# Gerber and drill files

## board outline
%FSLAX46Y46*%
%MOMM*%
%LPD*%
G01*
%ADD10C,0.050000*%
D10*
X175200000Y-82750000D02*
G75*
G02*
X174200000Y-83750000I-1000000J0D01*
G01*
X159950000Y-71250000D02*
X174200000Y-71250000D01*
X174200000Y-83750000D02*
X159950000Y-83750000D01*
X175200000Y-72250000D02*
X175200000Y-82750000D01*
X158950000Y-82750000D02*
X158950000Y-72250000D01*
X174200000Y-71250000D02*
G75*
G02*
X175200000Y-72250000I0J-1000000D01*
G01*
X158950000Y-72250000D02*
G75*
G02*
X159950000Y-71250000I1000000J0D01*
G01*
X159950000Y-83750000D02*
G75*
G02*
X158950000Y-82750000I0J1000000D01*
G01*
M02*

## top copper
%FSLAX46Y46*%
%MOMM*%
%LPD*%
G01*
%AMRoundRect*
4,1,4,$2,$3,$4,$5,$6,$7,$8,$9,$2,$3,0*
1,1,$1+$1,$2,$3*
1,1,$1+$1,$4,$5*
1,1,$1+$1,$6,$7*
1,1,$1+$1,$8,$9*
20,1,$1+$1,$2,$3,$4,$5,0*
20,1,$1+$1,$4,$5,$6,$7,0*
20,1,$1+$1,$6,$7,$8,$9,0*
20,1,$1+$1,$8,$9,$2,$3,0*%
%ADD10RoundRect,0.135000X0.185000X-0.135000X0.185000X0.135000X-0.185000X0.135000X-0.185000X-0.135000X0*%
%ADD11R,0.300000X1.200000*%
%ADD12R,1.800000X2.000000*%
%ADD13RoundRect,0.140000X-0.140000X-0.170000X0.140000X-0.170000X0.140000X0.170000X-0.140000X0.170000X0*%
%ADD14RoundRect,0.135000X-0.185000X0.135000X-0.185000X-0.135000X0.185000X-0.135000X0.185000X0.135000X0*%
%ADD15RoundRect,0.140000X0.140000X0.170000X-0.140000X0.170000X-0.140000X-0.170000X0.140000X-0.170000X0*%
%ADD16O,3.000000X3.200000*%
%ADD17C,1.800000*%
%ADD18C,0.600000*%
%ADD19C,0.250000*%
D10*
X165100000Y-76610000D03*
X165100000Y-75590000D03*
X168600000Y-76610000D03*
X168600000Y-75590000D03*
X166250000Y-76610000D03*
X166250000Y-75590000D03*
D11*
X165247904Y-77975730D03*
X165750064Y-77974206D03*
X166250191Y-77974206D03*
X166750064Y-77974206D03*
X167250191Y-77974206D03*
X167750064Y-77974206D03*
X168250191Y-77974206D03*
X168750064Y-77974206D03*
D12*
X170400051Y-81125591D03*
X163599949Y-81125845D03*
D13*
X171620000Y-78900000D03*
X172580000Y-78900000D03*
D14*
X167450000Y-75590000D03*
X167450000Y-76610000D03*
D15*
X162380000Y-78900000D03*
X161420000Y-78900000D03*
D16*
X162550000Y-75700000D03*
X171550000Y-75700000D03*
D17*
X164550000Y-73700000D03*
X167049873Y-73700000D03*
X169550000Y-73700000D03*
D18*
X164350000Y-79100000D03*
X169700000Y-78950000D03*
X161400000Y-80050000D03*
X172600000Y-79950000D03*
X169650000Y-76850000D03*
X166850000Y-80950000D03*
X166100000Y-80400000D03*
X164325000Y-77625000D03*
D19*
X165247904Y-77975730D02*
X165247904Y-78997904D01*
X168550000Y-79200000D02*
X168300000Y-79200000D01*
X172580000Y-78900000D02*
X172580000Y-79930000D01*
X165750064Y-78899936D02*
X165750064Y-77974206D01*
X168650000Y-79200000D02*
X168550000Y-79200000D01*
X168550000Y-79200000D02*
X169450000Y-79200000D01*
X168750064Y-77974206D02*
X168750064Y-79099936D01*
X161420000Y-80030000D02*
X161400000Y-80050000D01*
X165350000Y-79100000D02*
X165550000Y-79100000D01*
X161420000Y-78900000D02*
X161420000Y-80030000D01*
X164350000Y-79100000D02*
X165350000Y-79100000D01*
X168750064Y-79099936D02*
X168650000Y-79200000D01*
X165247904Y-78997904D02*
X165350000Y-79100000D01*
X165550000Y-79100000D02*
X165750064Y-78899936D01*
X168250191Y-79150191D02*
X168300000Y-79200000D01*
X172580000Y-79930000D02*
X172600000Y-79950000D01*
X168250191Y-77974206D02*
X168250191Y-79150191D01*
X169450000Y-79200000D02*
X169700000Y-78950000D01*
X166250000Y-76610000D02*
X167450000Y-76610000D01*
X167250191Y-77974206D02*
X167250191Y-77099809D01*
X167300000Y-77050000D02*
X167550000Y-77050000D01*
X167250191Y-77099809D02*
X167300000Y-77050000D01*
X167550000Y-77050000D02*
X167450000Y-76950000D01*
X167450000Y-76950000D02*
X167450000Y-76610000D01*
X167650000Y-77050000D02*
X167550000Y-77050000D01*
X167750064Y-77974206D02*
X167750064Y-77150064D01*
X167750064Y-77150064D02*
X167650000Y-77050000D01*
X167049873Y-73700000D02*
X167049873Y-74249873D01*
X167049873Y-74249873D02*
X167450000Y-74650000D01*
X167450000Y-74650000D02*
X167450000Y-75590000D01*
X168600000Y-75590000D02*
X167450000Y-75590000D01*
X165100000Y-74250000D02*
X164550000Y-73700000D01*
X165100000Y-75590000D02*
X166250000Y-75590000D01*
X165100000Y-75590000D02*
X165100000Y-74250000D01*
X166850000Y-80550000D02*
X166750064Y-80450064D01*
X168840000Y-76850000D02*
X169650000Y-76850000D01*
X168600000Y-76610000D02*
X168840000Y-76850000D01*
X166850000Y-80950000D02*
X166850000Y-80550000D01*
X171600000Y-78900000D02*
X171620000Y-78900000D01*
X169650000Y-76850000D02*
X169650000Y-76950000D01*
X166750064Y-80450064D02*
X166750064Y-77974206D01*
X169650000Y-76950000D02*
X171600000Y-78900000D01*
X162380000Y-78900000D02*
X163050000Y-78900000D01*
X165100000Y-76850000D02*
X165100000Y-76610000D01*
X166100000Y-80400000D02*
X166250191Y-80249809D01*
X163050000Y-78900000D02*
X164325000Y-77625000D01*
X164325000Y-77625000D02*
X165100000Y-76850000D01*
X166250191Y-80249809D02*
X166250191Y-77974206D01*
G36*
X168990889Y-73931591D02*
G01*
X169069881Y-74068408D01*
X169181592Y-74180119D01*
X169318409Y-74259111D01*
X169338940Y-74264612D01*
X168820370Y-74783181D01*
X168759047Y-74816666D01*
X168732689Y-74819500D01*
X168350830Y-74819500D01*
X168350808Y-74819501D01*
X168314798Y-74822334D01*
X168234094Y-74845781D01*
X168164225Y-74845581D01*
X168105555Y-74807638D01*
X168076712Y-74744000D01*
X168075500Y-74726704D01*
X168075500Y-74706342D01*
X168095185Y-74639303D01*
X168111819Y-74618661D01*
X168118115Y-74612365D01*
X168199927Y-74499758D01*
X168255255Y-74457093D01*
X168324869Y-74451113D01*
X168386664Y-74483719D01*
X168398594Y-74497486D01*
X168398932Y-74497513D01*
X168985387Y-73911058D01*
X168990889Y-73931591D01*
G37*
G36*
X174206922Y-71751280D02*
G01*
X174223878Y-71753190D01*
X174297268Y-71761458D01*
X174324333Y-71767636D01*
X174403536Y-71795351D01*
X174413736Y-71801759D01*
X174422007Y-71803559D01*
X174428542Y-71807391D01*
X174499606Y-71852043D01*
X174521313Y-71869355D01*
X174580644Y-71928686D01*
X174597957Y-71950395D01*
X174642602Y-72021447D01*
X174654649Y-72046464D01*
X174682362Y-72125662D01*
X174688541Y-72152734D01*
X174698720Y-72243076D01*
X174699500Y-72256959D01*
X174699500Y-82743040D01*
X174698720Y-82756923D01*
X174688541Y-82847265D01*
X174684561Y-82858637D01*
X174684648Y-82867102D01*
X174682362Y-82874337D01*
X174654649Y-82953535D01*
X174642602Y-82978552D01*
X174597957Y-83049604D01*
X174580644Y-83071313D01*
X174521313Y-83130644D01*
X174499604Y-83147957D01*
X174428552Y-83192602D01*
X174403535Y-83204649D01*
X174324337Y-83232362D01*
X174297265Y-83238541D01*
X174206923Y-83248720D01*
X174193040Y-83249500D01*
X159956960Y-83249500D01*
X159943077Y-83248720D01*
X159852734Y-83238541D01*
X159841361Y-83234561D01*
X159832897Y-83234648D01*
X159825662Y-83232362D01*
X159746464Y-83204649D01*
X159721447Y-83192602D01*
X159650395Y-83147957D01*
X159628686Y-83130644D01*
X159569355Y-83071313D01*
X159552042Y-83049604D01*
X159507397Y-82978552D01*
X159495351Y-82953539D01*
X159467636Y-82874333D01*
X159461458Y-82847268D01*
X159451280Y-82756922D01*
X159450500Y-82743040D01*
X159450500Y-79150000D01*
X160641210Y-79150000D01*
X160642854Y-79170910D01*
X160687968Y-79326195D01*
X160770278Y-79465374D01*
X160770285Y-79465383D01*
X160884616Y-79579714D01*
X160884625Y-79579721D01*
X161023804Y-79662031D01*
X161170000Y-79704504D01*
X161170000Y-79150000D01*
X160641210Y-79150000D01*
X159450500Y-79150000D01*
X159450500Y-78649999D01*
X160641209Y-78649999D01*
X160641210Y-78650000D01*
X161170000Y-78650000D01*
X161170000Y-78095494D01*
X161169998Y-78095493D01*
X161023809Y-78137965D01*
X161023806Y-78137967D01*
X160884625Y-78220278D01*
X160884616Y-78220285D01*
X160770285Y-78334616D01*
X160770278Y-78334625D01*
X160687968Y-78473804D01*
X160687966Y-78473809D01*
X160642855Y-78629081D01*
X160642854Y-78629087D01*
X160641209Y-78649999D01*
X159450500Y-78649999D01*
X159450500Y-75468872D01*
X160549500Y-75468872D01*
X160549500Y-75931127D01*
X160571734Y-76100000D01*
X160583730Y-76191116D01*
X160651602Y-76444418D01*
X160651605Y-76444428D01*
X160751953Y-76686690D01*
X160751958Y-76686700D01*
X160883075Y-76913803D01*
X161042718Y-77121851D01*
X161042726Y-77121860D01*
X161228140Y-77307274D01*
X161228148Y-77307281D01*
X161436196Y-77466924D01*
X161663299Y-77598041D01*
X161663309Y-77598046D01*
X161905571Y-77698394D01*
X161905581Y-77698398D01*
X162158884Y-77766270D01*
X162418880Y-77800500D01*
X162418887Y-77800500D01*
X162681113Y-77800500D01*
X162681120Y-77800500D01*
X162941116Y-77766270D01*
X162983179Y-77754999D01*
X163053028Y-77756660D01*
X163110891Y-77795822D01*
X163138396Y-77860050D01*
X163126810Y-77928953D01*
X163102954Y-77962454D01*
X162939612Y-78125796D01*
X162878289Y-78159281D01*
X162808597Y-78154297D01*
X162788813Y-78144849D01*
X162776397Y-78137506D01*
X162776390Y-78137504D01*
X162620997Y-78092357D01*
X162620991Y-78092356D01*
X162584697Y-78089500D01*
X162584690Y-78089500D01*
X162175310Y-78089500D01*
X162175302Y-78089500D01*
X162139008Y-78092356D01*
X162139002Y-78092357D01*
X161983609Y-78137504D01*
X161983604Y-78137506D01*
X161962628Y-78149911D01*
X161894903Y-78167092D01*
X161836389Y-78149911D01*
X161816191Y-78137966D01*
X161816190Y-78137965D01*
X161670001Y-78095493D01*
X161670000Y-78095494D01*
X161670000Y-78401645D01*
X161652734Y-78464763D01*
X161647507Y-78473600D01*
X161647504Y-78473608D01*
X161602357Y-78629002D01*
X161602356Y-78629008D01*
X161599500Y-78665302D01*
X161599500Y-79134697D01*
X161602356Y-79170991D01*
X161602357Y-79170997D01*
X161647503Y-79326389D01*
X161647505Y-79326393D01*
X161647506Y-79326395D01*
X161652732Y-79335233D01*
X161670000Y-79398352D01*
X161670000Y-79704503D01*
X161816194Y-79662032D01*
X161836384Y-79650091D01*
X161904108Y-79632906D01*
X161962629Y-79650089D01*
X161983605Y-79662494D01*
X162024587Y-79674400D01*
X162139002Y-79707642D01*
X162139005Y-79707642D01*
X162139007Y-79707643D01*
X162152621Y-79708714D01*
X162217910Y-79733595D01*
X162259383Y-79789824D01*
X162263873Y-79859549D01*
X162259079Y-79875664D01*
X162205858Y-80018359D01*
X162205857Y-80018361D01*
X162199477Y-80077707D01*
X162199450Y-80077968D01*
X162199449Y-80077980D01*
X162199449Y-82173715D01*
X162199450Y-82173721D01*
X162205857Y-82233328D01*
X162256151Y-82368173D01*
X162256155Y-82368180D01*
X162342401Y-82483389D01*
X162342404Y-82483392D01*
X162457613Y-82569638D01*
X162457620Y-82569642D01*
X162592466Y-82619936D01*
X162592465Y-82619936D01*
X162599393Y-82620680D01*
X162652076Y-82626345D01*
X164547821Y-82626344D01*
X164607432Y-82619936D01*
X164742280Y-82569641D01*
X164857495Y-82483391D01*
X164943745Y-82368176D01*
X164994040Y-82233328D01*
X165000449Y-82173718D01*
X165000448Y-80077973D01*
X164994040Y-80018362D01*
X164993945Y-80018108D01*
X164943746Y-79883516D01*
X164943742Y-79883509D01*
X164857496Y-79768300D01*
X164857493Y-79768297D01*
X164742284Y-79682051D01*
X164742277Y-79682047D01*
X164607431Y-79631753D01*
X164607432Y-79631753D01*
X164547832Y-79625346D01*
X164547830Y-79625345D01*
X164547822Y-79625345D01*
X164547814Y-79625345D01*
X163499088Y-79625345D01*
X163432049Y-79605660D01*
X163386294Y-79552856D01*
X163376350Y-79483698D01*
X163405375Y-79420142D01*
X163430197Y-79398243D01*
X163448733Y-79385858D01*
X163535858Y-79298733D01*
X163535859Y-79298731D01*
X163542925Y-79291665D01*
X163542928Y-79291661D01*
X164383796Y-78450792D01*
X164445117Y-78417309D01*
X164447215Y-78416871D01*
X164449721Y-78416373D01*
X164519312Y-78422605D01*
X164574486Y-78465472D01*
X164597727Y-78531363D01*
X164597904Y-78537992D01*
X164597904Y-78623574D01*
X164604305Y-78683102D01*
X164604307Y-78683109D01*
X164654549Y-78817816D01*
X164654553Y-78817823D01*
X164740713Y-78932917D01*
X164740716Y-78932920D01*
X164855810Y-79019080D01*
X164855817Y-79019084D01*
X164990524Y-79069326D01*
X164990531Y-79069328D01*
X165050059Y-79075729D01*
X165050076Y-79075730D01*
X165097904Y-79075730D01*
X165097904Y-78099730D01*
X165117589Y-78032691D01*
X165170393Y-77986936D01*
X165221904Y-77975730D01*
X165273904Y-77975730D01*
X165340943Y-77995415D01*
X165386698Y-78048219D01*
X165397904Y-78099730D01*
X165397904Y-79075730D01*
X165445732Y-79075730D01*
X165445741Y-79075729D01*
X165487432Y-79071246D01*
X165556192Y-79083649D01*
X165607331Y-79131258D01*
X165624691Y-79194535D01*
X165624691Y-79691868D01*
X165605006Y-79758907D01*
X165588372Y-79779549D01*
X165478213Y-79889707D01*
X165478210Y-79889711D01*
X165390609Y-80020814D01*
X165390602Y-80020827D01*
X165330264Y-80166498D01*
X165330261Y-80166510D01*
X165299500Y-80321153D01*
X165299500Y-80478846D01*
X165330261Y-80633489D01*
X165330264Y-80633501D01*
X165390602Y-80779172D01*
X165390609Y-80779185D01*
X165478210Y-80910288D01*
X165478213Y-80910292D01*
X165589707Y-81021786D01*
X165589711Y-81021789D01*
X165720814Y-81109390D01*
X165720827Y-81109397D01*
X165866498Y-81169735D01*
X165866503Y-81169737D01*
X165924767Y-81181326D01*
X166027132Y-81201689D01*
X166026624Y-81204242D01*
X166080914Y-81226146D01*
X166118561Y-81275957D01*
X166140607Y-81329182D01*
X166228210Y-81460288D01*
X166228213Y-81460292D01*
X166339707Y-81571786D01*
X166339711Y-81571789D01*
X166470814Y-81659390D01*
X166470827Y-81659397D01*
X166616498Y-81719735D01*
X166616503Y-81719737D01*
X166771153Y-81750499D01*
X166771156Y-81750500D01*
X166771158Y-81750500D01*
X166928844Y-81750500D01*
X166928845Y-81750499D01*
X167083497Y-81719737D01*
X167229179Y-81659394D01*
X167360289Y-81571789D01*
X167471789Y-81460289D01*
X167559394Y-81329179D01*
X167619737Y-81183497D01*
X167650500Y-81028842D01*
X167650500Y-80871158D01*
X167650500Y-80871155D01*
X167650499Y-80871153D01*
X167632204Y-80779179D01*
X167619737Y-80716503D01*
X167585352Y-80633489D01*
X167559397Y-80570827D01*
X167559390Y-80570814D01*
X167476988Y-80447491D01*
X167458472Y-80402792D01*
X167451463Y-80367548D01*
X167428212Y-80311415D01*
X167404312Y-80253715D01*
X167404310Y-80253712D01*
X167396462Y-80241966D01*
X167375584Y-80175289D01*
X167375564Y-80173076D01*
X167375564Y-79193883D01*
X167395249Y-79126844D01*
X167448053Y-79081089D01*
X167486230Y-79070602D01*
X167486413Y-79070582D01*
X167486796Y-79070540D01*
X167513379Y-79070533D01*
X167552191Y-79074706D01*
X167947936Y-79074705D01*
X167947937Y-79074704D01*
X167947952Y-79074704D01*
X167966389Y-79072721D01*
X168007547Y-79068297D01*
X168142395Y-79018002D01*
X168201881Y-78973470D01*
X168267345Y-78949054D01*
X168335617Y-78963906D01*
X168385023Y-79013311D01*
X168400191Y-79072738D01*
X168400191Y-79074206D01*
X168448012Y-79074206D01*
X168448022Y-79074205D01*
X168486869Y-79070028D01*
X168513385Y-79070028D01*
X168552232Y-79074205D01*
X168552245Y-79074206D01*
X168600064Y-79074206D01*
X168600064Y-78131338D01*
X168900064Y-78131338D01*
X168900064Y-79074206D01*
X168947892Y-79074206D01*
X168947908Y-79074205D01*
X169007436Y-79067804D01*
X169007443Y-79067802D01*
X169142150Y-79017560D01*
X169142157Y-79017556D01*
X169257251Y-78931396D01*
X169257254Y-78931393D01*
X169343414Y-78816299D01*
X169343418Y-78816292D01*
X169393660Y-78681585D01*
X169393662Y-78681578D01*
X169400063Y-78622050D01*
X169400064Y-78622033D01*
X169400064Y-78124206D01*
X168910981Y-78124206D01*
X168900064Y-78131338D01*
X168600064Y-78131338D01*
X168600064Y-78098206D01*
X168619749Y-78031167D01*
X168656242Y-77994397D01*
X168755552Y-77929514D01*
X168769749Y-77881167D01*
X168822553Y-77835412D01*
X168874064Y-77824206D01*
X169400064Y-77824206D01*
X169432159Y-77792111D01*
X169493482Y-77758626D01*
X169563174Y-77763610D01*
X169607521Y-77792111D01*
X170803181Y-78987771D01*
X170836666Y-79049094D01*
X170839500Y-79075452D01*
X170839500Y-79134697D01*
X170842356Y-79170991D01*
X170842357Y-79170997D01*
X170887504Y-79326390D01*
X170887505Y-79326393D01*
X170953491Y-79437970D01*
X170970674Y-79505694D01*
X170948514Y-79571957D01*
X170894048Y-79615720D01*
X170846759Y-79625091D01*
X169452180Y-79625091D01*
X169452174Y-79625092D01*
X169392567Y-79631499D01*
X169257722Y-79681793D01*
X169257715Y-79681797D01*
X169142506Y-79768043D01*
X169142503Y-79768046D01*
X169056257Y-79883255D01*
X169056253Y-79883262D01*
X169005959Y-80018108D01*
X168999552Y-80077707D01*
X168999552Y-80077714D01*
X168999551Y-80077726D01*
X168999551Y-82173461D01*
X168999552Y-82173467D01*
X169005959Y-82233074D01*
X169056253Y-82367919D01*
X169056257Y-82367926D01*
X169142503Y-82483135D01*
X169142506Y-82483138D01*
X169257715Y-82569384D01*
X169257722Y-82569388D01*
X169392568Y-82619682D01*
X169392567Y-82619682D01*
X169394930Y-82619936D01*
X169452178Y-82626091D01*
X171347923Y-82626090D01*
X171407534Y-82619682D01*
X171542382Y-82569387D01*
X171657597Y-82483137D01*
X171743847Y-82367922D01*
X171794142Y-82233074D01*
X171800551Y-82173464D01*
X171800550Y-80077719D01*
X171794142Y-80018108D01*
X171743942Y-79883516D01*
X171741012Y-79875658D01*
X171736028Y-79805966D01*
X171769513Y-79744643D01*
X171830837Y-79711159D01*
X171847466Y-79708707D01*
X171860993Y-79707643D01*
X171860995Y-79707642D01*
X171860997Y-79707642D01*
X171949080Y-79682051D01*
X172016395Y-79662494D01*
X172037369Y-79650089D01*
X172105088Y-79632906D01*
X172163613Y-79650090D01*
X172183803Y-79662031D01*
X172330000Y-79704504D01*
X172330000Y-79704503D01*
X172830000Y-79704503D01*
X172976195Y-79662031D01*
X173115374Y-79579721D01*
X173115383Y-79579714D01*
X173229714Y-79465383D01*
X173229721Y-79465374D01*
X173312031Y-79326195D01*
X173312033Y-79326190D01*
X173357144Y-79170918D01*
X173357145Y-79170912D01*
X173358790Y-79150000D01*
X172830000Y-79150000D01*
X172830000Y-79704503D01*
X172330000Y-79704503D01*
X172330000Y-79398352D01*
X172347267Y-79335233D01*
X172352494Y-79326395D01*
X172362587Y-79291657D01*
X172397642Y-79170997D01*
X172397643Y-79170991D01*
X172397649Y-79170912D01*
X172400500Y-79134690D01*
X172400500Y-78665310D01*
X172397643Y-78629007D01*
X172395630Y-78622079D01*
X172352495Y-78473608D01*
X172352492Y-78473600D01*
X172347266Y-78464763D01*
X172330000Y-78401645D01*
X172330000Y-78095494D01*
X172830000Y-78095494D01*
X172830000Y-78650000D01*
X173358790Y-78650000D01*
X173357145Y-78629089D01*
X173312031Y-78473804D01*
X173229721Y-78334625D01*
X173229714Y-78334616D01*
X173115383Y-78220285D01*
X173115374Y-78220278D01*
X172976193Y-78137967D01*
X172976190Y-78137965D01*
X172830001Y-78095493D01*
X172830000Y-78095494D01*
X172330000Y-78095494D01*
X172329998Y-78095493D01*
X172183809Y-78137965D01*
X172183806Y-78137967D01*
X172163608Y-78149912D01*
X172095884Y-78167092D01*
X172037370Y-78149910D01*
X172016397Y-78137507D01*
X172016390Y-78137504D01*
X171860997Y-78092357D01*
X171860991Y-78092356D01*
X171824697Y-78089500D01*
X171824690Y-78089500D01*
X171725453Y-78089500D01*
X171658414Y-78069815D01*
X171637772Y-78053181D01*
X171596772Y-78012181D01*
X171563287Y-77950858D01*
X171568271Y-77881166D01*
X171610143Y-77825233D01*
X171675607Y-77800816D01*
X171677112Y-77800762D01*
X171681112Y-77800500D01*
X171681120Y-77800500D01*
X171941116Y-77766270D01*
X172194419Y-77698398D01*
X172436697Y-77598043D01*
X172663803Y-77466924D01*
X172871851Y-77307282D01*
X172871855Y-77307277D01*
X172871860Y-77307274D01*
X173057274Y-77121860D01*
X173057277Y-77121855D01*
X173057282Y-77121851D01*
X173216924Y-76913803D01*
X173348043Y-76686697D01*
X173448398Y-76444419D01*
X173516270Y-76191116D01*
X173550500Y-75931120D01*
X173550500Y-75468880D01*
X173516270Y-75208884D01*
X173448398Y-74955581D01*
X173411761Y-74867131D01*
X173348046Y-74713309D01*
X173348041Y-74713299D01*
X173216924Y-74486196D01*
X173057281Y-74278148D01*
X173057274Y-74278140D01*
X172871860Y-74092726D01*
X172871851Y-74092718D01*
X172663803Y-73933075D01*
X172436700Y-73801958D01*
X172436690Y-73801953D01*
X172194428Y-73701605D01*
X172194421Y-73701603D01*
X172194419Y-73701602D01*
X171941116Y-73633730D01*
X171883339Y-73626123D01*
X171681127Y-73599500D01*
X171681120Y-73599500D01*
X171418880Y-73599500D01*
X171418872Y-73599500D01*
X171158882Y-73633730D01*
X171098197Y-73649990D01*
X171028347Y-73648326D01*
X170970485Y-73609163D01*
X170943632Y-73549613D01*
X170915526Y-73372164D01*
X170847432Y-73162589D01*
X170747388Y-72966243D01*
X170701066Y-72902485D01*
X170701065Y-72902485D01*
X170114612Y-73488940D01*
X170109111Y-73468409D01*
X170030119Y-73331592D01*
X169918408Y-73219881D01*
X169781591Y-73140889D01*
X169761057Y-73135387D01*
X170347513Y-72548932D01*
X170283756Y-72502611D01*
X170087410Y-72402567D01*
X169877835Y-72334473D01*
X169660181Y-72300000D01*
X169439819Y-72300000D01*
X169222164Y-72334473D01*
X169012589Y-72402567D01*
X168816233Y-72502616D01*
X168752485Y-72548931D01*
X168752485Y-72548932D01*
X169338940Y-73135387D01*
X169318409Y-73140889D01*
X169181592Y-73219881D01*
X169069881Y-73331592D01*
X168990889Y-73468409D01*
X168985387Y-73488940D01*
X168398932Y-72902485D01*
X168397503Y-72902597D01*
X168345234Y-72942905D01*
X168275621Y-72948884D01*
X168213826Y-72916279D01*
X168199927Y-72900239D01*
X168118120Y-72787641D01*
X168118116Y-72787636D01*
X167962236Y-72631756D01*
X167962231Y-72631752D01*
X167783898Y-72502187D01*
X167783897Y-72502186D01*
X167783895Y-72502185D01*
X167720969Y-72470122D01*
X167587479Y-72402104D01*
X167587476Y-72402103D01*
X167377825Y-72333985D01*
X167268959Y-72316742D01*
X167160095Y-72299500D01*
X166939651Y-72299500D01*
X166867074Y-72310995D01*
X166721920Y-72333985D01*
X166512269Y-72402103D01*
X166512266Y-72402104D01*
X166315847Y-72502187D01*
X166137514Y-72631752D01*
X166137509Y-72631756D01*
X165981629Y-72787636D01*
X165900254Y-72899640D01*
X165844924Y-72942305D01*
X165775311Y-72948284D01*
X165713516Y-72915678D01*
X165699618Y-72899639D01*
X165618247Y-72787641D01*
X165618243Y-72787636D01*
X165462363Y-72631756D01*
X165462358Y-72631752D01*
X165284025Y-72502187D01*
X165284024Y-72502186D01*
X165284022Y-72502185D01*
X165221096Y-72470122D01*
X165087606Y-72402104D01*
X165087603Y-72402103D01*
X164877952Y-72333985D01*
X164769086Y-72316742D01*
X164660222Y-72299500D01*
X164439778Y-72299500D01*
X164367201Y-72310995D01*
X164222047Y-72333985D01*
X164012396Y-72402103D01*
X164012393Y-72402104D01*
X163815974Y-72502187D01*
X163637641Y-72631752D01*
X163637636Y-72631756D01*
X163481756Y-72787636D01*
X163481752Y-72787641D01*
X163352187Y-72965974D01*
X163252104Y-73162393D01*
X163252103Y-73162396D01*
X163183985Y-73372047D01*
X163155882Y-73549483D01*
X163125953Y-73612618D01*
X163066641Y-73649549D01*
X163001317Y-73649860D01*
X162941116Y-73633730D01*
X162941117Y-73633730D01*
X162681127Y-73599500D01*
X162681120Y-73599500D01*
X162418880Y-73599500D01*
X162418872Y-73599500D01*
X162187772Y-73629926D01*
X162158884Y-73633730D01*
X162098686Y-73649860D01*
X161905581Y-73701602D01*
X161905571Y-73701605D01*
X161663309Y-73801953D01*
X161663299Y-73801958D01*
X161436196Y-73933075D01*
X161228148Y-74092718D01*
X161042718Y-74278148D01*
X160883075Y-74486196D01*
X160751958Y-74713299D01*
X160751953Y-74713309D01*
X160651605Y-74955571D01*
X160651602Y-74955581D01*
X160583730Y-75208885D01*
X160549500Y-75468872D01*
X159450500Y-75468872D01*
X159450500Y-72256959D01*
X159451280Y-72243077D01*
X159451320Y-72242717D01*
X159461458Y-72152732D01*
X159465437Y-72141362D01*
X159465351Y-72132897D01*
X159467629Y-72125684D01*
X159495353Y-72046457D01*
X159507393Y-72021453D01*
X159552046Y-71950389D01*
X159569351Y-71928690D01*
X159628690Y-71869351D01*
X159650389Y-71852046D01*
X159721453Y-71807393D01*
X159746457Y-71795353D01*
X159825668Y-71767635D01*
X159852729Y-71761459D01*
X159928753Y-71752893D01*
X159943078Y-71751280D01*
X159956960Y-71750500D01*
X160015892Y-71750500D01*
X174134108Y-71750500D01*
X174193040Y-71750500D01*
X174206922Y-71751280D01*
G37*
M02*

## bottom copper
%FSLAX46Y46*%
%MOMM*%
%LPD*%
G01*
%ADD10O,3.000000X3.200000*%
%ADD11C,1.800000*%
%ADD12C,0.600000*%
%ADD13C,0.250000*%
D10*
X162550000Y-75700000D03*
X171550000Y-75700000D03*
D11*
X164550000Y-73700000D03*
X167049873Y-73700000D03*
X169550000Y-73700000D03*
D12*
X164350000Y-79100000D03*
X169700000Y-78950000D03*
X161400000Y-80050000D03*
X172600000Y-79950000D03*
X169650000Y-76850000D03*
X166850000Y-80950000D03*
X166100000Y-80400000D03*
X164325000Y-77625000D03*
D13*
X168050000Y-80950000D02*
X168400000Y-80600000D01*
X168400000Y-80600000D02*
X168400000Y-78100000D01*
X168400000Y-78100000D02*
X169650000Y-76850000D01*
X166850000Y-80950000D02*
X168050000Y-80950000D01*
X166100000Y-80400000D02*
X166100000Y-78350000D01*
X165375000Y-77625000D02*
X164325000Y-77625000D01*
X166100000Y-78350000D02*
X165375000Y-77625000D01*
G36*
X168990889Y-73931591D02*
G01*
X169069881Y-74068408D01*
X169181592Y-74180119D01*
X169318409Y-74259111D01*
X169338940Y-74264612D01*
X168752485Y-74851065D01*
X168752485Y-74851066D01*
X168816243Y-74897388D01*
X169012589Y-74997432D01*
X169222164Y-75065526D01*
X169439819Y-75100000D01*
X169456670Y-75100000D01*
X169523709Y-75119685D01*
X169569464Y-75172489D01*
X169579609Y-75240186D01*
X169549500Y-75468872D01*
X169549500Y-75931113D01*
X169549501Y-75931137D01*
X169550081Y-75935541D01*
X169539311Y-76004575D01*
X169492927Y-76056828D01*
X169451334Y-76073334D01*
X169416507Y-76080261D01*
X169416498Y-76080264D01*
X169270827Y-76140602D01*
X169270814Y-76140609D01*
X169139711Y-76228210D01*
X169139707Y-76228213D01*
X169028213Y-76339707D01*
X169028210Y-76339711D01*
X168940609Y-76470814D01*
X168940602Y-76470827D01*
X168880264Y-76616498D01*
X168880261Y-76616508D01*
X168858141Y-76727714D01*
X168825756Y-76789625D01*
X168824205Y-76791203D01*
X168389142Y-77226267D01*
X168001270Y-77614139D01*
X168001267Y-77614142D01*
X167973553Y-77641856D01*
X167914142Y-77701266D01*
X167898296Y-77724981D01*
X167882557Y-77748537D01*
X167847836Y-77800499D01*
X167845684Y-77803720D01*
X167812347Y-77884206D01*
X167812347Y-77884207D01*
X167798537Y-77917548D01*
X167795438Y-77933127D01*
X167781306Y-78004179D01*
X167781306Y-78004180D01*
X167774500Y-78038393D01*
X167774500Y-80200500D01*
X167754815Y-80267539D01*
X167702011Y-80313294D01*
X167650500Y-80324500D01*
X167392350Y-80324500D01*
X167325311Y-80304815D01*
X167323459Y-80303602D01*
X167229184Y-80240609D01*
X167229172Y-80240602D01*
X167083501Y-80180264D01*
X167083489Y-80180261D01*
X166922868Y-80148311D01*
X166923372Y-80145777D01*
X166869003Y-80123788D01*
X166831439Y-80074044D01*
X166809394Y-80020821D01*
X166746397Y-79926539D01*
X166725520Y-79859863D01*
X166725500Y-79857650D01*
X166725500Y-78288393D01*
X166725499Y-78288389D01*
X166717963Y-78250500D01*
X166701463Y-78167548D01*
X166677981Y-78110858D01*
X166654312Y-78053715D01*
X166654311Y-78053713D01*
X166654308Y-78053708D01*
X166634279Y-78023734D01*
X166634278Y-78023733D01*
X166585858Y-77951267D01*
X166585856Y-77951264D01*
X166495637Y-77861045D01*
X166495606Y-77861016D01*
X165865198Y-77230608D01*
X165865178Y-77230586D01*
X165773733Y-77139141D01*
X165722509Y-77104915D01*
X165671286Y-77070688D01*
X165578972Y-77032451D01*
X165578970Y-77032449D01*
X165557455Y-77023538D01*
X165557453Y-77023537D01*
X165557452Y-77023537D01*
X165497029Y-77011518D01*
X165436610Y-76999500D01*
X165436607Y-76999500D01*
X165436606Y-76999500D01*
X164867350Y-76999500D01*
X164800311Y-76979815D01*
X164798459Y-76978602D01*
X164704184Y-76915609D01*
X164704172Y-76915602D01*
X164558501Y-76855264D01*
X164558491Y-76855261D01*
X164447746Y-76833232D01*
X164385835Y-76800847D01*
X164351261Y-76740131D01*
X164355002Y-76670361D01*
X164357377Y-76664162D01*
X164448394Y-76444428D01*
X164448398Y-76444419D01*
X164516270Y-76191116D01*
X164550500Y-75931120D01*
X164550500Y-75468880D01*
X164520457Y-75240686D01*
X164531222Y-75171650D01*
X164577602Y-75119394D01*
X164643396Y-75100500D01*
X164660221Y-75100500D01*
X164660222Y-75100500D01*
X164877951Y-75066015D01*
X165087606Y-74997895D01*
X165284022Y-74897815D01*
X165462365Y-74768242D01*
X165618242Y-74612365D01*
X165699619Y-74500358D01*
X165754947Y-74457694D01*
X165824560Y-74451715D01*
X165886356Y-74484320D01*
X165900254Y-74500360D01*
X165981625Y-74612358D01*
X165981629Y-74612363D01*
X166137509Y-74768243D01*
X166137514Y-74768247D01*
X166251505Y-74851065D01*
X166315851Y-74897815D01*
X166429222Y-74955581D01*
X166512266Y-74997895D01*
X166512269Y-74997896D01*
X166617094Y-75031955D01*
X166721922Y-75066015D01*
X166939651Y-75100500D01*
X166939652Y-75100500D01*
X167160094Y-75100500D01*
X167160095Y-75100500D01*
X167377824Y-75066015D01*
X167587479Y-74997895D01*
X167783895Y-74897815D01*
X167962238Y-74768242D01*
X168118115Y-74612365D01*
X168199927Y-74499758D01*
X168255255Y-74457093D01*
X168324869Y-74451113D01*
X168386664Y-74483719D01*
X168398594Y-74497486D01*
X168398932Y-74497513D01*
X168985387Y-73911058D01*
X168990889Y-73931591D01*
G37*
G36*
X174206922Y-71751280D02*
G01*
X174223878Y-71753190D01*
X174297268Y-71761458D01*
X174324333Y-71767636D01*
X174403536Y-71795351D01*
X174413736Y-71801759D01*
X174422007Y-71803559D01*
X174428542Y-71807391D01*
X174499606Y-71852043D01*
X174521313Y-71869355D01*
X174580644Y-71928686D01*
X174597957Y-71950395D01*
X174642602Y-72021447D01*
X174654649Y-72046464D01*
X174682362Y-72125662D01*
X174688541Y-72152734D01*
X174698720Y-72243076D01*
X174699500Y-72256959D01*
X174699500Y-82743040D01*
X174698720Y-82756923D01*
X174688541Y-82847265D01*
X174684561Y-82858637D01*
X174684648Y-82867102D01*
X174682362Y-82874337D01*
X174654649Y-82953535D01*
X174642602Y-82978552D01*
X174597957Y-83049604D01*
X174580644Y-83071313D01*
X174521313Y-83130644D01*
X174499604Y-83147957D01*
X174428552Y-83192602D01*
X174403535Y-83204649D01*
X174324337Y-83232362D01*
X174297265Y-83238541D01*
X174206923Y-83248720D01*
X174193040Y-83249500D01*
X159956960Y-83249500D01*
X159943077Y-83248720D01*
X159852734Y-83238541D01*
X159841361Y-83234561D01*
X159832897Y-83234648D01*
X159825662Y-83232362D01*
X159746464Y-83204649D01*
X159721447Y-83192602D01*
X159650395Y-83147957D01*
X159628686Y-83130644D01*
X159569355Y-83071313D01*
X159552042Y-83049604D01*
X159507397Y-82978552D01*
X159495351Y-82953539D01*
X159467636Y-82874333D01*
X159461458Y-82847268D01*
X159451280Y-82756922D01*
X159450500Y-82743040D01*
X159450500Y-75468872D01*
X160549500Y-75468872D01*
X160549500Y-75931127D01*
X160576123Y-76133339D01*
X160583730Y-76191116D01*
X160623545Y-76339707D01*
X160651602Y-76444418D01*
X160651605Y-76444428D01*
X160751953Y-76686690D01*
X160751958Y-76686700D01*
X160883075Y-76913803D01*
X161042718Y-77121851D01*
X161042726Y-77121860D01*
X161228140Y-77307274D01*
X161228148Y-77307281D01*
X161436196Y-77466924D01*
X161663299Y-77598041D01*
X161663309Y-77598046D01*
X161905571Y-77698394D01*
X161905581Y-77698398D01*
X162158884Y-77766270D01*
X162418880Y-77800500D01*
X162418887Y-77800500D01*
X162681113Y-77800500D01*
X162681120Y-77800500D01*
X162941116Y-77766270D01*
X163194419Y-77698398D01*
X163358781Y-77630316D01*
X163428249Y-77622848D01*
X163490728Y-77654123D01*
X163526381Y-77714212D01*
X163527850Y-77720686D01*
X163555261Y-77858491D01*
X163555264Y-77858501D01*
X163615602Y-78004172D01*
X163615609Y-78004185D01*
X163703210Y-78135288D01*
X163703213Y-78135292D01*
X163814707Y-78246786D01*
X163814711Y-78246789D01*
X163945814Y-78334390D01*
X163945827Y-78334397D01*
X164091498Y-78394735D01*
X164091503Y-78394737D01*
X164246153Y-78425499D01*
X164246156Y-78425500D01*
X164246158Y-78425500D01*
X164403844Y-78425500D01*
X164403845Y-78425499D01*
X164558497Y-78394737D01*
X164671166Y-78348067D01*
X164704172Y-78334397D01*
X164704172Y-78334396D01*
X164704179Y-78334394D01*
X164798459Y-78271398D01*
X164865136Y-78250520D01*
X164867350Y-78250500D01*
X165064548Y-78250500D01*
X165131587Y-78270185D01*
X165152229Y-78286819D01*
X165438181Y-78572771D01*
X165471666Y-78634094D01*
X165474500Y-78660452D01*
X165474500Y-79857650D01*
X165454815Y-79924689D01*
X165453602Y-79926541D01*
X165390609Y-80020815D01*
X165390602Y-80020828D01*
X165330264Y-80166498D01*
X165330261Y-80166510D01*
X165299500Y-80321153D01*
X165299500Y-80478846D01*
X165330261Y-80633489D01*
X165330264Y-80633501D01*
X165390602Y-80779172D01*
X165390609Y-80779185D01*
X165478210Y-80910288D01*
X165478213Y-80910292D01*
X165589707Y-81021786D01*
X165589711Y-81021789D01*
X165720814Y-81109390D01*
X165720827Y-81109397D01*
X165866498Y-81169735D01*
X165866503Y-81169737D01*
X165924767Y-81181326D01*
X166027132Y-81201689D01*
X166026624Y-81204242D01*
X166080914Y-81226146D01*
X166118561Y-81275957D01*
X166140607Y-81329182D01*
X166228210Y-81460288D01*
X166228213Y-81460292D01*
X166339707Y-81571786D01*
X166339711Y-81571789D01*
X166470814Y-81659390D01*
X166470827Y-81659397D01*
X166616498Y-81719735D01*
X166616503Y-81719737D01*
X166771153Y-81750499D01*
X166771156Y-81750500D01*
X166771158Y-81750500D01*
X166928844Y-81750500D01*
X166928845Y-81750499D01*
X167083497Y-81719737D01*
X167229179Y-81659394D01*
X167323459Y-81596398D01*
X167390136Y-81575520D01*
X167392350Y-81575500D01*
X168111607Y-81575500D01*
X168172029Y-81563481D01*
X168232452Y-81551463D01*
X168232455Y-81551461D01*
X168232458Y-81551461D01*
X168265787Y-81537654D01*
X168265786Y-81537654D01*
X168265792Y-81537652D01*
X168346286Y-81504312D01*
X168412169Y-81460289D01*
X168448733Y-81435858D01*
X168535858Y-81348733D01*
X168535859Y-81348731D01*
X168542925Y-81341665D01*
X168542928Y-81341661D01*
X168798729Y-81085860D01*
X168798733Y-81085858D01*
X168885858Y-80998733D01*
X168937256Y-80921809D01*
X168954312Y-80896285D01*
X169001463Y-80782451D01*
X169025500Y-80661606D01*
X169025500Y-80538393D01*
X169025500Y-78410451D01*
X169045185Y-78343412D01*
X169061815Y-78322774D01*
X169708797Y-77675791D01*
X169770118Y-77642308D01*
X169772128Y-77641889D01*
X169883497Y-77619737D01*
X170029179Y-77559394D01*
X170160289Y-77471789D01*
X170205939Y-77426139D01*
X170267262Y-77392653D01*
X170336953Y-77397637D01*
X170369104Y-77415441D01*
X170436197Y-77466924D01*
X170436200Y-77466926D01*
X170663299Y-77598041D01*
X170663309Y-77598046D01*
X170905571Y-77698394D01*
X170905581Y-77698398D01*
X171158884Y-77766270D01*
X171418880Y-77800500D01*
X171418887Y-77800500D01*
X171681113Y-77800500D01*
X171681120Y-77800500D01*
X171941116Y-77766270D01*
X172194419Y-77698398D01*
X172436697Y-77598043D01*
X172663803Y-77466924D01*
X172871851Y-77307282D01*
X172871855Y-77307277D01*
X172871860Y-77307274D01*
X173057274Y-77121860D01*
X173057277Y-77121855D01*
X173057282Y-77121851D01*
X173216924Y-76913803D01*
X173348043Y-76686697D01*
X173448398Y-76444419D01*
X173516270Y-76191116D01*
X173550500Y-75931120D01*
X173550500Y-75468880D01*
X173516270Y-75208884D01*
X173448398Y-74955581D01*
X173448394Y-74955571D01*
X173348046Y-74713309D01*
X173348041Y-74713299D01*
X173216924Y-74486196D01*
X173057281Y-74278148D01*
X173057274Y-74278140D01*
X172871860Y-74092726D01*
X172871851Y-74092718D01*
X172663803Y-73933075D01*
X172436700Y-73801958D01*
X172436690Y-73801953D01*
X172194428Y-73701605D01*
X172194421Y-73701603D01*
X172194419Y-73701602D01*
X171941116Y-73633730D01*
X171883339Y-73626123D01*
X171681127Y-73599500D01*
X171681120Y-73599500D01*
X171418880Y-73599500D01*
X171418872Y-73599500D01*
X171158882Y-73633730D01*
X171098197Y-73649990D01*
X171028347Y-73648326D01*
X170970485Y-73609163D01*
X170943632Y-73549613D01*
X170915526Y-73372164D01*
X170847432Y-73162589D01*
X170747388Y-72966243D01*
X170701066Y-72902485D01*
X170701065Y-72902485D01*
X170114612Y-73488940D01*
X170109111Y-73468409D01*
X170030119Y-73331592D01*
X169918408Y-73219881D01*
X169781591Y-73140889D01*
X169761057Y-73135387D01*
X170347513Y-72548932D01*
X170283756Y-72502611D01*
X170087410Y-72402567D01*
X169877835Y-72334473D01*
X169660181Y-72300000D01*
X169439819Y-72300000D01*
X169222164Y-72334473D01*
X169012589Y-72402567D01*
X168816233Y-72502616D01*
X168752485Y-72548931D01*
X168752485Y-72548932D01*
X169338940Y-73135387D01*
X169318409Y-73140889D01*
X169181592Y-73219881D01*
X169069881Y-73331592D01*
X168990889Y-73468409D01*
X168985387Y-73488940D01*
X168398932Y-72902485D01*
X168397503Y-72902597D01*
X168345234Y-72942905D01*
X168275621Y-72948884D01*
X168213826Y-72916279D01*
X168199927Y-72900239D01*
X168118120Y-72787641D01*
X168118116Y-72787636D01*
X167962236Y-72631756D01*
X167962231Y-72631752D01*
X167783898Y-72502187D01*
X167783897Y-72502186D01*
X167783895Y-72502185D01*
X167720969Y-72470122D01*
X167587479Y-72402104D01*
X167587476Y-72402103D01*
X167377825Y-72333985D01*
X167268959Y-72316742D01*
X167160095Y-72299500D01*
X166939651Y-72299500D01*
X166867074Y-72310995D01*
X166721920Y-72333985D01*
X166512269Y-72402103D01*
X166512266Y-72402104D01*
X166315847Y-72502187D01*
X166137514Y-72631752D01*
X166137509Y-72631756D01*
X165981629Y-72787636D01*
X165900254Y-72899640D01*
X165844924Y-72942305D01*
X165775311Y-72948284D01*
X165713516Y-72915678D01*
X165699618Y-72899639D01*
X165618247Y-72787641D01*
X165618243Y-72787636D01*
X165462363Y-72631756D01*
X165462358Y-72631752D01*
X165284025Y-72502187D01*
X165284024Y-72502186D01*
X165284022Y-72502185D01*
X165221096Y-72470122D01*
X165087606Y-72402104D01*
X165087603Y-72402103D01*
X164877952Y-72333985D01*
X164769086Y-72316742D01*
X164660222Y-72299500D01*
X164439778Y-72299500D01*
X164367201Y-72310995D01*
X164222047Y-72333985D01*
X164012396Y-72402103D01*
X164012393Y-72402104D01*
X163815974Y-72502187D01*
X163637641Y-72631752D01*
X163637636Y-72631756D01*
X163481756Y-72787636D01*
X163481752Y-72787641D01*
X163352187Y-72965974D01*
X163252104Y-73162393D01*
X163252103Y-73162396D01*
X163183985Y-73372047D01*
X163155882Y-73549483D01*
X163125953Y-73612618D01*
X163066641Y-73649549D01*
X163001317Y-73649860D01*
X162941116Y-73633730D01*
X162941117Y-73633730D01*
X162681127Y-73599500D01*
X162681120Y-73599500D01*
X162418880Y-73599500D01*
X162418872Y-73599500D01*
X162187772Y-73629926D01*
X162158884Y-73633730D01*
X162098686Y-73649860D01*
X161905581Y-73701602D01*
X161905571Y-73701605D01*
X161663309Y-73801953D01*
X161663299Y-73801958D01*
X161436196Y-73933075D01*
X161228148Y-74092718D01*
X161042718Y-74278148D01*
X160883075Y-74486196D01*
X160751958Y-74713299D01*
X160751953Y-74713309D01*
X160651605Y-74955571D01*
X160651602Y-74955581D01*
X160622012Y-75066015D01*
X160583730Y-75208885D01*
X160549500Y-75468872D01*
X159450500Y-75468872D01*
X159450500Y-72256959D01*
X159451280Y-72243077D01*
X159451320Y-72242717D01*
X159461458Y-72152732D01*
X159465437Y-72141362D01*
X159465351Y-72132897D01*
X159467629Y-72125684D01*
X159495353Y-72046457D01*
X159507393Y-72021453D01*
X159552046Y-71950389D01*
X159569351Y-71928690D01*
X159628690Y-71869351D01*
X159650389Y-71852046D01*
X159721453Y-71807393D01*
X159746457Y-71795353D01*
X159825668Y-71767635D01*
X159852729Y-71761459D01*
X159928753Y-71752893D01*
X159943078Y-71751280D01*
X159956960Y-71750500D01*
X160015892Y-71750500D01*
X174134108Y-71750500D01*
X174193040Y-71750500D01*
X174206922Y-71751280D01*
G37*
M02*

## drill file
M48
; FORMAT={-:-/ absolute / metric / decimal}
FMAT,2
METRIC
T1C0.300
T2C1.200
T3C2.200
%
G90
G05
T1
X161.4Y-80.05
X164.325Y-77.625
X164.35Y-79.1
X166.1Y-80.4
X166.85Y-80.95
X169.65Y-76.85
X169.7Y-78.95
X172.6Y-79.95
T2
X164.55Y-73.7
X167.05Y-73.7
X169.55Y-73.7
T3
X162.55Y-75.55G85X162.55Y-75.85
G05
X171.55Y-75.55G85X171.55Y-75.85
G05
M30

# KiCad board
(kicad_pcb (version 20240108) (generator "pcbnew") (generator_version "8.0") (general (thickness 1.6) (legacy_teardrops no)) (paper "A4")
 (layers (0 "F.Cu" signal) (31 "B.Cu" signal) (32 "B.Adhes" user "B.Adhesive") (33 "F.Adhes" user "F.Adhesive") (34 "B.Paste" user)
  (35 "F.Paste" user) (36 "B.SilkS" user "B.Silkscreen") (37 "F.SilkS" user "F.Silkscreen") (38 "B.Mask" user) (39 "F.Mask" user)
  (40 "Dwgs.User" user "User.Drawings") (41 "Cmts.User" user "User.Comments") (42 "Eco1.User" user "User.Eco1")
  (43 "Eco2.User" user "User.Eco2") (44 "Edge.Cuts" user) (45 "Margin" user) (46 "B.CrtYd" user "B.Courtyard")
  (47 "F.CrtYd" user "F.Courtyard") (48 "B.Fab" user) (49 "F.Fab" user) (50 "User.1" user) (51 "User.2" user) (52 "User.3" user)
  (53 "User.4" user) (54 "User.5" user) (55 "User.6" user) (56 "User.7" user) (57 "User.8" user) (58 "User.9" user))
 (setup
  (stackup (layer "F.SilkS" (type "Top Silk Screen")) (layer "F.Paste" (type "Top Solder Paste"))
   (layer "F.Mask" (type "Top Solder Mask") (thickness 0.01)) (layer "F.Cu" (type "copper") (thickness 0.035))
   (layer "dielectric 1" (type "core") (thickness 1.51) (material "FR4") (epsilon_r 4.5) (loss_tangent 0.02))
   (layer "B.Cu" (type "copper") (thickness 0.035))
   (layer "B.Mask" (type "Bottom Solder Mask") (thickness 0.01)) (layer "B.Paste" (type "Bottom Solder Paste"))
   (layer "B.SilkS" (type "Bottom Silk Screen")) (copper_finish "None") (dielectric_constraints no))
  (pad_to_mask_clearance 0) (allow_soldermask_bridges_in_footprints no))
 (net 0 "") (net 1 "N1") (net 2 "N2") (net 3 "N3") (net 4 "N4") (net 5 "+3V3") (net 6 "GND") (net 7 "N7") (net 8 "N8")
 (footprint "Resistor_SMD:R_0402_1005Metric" (layer "F.Cu") (at 165.1 76.1 90)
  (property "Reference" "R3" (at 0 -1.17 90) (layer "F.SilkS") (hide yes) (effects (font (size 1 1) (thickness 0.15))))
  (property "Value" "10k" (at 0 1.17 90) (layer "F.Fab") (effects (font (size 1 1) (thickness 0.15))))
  (pad "1" smd roundrect (at -0.51 0 90) (size 0.54 0.64) (layers "F.Cu" "F.Paste" "F.Mask") (roundrect_rratio 0.25) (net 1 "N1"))
  (pad "2" smd roundrect (at 0.51 0 90) (size 0.54 0.64) (layers "F.Cu" "F.Paste" "F.Mask") (roundrect_rratio 0.25) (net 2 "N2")))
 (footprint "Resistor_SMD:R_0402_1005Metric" (layer "F.Cu") (at 168.6 76.1 90)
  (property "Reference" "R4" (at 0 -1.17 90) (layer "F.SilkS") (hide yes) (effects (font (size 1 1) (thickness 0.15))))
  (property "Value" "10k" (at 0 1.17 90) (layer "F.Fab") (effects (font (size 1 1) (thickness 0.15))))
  (pad "1" smd roundrect (at -0.51 0 90) (size 0.54 0.64) (layers "F.Cu" "F.Paste" "F.Mask") (roundrect_rratio 0.25) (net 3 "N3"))
  (pad "2" smd roundrect (at 0.51 0 90) (size 0.54 0.64) (layers "F.Cu" "F.Paste" "F.Mask") (roundrect_rratio 0.25) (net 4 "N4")))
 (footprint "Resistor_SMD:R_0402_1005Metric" (layer "F.Cu") (at 166.25 76.1 90)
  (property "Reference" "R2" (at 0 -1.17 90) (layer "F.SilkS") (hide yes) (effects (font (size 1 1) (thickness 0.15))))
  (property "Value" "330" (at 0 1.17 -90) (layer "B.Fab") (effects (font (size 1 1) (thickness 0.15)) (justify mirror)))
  (pad "1" smd roundrect (at -0.51 0 90) (size 0.54 0.64) (layers "F.Cu" "F.Paste" "F.Mask") (roundrect_rratio 0.25) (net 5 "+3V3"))
  (pad "2" smd roundrect (at 0.51 0 90) (size 0.54 0.64) (layers "F.Cu" "F.Paste" "F.Mask") (roundrect_rratio 0.25) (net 2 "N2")))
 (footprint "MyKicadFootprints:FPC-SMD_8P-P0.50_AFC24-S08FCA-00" (layer "F.Cu") (at 167 79.55)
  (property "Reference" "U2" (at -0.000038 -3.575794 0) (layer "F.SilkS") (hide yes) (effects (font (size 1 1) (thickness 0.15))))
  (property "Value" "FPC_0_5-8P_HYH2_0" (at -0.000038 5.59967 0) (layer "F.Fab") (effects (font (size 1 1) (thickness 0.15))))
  (pad "1" smd rect (at -1.752096 -1.57427) (size 0.3 1.2) (layers "F.Cu" "F.Paste" "F.Mask") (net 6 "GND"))
  (pad "2" smd rect (at -1.249936 -1.575794) (size 0.3 1.2) (layers "F.Cu" "F.Paste" "F.Mask") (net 6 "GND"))
  (pad "3" smd rect (at -0.749809 -1.575794) (size 0.3 1.2) (layers "F.Cu" "F.Paste" "F.Mask") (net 1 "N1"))
  (pad "4" smd rect (at -0.249936 -1.575794) (size 0.3 1.2) (layers "F.Cu" "F.Paste" "F.Mask") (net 3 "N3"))
  (pad "5" smd rect (at 0.250191 -1.575794) (size 0.3 1.2) (layers "F.Cu" "F.Paste" "F.Mask") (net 5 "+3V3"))
  (pad "6" smd rect (at 0.750064 -1.575794) (size 0.3 1.2) (layers "F.Cu" "F.Paste" "F.Mask") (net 5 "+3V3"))
  (pad "7" smd rect (at 1.250191 -1.575794) (size 0.3 1.2) (layers "F.Cu" "F.Paste" "F.Mask") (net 6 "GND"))
  (pad "8" smd rect (at 1.750064 -1.575794) (size 0.3 1.2) (layers "F.Cu" "F.Paste" "F.Mask") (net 6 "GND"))
  (pad "9" smd rect (at 3.400051 1.575591 90) (size 2 1.8) (layers "F.Cu" "F.Paste" "F.Mask") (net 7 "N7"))
  (pad "10" smd rect (at -3.400051 1.575845 90) (size 2 1.8) (layers "F.Cu" "F.Paste" "F.Mask") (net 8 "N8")))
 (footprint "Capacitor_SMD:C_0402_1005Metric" (layer "F.Cu") (at 172.1 78.9)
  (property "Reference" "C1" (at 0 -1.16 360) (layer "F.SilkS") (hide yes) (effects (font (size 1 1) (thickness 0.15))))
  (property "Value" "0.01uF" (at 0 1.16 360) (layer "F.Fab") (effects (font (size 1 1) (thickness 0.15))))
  (pad "1" smd roundrect (at -0.48 0) (size 0.56 0.62) (layers "F.Cu" "F.Paste" "F.Mask") (roundrect_rratio 0.25) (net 3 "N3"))
  (pad "2" smd roundrect (at 0.48 0) (size 0.56 0.62) (layers "F.Cu" "F.Paste" "F.Mask") (roundrect_rratio 0.25) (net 6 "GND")))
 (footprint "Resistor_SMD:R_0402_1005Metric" (layer "F.Cu") (at 167.45 76.1 -90)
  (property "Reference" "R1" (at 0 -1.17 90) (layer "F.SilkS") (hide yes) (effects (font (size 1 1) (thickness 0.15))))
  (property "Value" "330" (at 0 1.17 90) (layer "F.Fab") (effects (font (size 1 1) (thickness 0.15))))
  (pad "1" smd roundrect (at -0.51 0 270) (size 0.54 0.64) (layers "F.Cu" "F.Paste" "F.Mask") (roundrect_rratio 0.25) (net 4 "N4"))
  (pad "2" smd roundrect (at 0.51 0 270) (size 0.54 0.64) (layers "F.Cu" "F.Paste" "F.Mask") (roundrect_rratio 0.25) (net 5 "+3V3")))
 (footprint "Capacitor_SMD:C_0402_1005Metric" (layer "F.Cu") (at 161.9 78.9 180)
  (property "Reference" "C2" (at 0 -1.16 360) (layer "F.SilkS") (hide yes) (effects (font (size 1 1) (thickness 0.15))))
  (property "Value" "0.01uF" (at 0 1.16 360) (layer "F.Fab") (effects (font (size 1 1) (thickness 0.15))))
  (pad "1" smd roundrect (at -0.48 0 180) (size 0.56 0.62) (layers "F.Cu" "F.Paste" "F.Mask") (roundrect_rratio 0.25) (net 1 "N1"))
  (pad "2" smd roundrect (at 0.48 0 180) (size 0.56 0.62) (layers "F.Cu" "F.Paste" "F.Mask") (roundrect_rratio 0.25) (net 6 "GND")))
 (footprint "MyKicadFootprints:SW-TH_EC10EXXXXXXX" (layer "B.Cu") (at 167.05 74.7)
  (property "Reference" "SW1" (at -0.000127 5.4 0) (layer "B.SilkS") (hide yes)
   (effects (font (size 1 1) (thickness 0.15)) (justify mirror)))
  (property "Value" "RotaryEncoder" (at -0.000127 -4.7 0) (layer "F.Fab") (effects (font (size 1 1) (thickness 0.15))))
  (pad "4" thru_hole oval (at -4.5 1 270) (size 3.2 3) (drill oval 2.500025 2.2) (layers "*.Cu" "*.Mask") (remove_unused_layers no))
  (pad "5" thru_hole oval (at 4.5 1 270) (size 3.2 3) (drill oval 2.500025 2.2) (layers "*.Cu" "*.Mask") (remove_unused_layers no))
  (pad "A" thru_hole circle (at -2.5 -1) (size 1.8 1.8) (drill 1.2) (layers "*.Cu" "*.Mask") (remove_unused_layers no) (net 2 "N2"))
  (pad "B" thru_hole circle (at -0.000127 -1) (size 1.8 1.8) (drill 1.2) (layers "*.Cu" "*.Mask") (remove_unused_layers no) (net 4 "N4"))
  (pad "C" thru_hole circle (at 2.5 -1) (size 1.8 1.8) (drill 1.2) (layers "*.Cu" "*.Mask") (remove_unused_layers no) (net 6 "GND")))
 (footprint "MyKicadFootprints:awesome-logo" (layer "B.Cu") (at 172.25 80.75 180)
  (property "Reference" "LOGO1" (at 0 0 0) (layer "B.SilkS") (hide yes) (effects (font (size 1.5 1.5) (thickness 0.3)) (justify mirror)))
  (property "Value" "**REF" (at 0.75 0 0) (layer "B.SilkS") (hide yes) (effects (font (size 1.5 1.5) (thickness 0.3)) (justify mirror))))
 (gr_arc (start 175.2 82.75) (mid 174.907107 83.457107) (end 174.2 83.75) (stroke (width 0.05) (type default)) (layer "Edge.Cuts"))
 (gr_line (start 159.95 71.25) (end 174.2 71.25) (stroke (width 0.05) (type default)) (layer "Edge.Cuts"))
 (gr_line (start 174.2 83.75) (end 159.95 83.75) (stroke (width 0.05) (type default)) (layer "Edge.Cuts"))
 (gr_line (start 175.2 72.25) (end 175.2 82.75) (stroke (width 0.05) (type default)) (layer "Edge.Cuts"))
 (gr_line (start 158.95 82.75) (end 158.95 72.25) (stroke (width 0.05) (type default)) (layer "Edge.Cuts"))
 (gr_arc (start 174.2 71.25) (mid 174.907107 71.542893) (end 175.2 72.25) (stroke (width 0.05) (type default)) (layer "Edge.Cuts"))
 (gr_arc (start 158.95 72.25) (mid 159.242893 71.542893) (end 159.95 71.25) (stroke (width 0.05) (type default)) (layer "Edge.Cuts"))
 (gr_arc (start 159.95 83.75) (mid 159.242893 83.457107) (end 158.95 82.75) (stroke (width 0.05) (type default)) (layer "Edge.Cuts"))
 (segment (start 165.247904 77.97573) (end 165.247904 78.997904) (width 0.25) (layer "F.Cu") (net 6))
 (segment (start 168.55 79.2) (end 168.3 79.2) (width 0.25) (layer "F.Cu") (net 6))
 (segment (start 172.58 78.9) (end 172.58 79.93) (width 0.25) (layer "F.Cu") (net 6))
 (segment (start 165.750064 78.899936) (end 165.750064 77.974206) (width 0.25) (layer "F.Cu") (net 6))
 (segment (start 168.65 79.2) (end 168.55 79.2) (width 0.25) (layer "F.Cu") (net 6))
 (segment (start 168.55 79.2) (end 169.45 79.2) (width 0.25) (layer "F.Cu") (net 6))
 (segment (start 168.750064 77.974206) (end 168.750064 79.099936) (width 0.25) (layer "F.Cu") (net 6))
 (segment (start 161.42 80.03) (end 161.4 80.05) (width 0.25) (layer "F.Cu") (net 6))
 (segment (start 165.35 79.1) (end 165.55 79.1) (width 0.25) (layer "F.Cu") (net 6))
 (segment (start 161.42 78.9) (end 161.42 80.03) (width 0.25) (layer "F.Cu") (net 6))
 (segment (start 164.35 79.1) (end 165.35 79.1) (width 0.25) (layer "F.Cu") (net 6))
 (segment (start 168.750064 79.099936) (end 168.65 79.2) (width 0.25) (layer "F.Cu") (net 6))
 (segment (start 165.247904 78.997904) (end 165.35 79.1) (width 0.25) (layer "F.Cu") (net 6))
 (segment (start 165.55 79.1) (end 165.750064 78.899936) (width 0.25) (layer "F.Cu") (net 6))
 (segment (start 168.250191 79.150191) (end 168.3 79.2) (width 0.25) (layer "F.Cu") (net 6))
 (segment (start 172.58 79.93) (end 172.6 79.95) (width 0.25) (layer "F.Cu") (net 6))
 (segment (start 168.250191 77.974206) (end 168.250191 79.150191) (width 0.25) (layer "F.Cu") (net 6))
 (segment (start 169.45 79.2) (end 169.7 78.95) (width 0.25) (layer "F.Cu") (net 6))
 (via (at 164.35 79.1) (size 0.6) (drill 0.3) (layers "F.Cu" "B.Cu") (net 6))
 (via (at 169.7 78.95) (size 0.6) (drill 0.3) (layers "F.Cu" "B.Cu") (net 6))
 (via (at 161.4 80.05) (size 0.6) (drill 0.3) (layers "F.Cu" "B.Cu") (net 6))
 (via (at 172.6 79.95) (size 0.6) (drill 0.3) (layers "F.Cu" "B.Cu") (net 6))
 (segment (start 166.25 76.61) (end 167.45 76.61) (width 0.25) (layer "F.Cu") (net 5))
 (segment (start 167.250191 77.974206) (end 167.250191 77.099809) (width 0.25) (layer "F.Cu") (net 5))
 (segment (start 167.3 77.05) (end 167.55 77.05) (width 0.25) (layer "F.Cu") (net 5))
 (segment (start 167.250191 77.099809) (end 167.3 77.05) (width 0.25) (layer "F.Cu") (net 5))
 (segment (start 167.55 77.05) (end 167.45 76.95) (width 0.25) (layer "F.Cu") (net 5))
 (segment (start 167.45 76.95) (end 167.45 76.61) (width 0.25) (layer "F.Cu") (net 5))
 (segment (start 167.65 77.05) (end 167.55 77.05) (width 0.25) (layer "F.Cu") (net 5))
 (segment (start 167.750064 77.974206) (end 167.750064 77.150064) (width 0.25) (layer "F.Cu") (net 5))
 (segment (start 167.750064 77.150064) (end 167.65 77.05) (width 0.25) (layer "F.Cu") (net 5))
 (segment (start 167.049873 73.7) (end 167.049873 74.249873) (width 0.25) (layer "F.Cu") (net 4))
 (segment (start 167.049873 74.249873) (end 167.45 74.65) (width 0.25) (layer "F.Cu") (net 4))
 (segment (start 167.45 74.65) (end 167.45 75.59) (width 0.25) (layer "F.Cu") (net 4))
 (segment (start 168.6 75.59) (end 167.45 75.59) (width 0.25) (layer "F.Cu") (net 4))
 (segment (start 165.1 74.25) (end 164.55 73.7) (width 0.25) (layer "F.Cu") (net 2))
 (segment (start 165.1 75.59) (end 166.25 75.59) (width 0.25) (layer "F.Cu") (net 2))
 (segment (start 165.1 75.59) (end 165.1 74.25) (width 0.25) (layer "F.Cu") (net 2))
 (segment (start 166.85 80.55) (end 166.750064 80.450064) (width 0.25) (layer "F.Cu") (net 3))
 (segment (start 168.84 76.85) (end 169.65 76.85) (width 0.25) (layer "F.Cu") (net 3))
 (segment (start 168.6 76.61) (end 168.84 76.85) (width 0.25) (layer "F.Cu") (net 3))
 (segment (start 166.85 80.95) (end 166.85 80.55) (width 0.25) (layer "F.Cu") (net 3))
 (segment (start 171.6 78.9) (end 171.62 78.9) (width 0.25) (layer "F.Cu") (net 3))
 (segment (start 169.65 76.85) (end 169.65 76.95) (width 0.25) (layer "F.Cu") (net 3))
 (segment (start 166.750064 80.450064) (end 166.750064 77.974206) (width 0.25) (layer "F.Cu") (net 3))
 (segment (start 169.65 76.95) (end 171.6 78.9) (width 0.25) (layer "F.Cu") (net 3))
 (via (at 169.65 76.85) (size 0.6) (drill 0.3) (layers "F.Cu" "B.Cu") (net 3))
 (via (at 166.85 80.95) (size 0.6) (drill 0.3) (layers "F.Cu" "B.Cu") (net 3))
 (segment (start 168.05 80.95) (end 168.4 80.6) (width 0.25) (layer "B.Cu") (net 3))
 (segment (start 168.4 80.6) (end 168.4 78.1) (width 0.25) (layer "B.Cu") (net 3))
 (segment (start 168.4 78.1) (end 169.65 76.85) (width 0.25) (layer "B.Cu") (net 3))
 (segment (start 166.85 80.95) (end 168.05 80.95) (width 0.25) (layer "B.Cu") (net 3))
 (segment (start 162.38 78.9) (end 163.05 78.9) (width 0.25) (layer "F.Cu") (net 1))
 (segment (start 165.1 76.85) (end 165.1 76.61) (width 0.25) (layer "F.Cu") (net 1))
 (segment (start 166.1 80.4) (end 166.250191 80.249809) (width 0.25) (layer "F.Cu") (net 1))
 (segment (start 163.05 78.9) (end 164.325 77.625) (width 0.25) (layer "F.Cu") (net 1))
 (segment (start 164.325 77.625) (end 165.1 76.85) (width 0.25) (layer "F.Cu") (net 1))
 (segment (start 166.250191 80.249809) (end 166.250191 77.974206) (width 0.25) (layer "F.Cu") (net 1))
 (via (at 166.1 80.4) (size 0.6) (drill 0.3) (layers "F.Cu" "B.Cu") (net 1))
 (via (at 164.325 77.625) (size 0.6) (drill 0.3) (layers "F.Cu" "B.Cu") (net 1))
 (segment (start 166.1 80.4) (end 166.1 78.35) (width 0.25) (layer "B.Cu") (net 1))
 (segment (start 165.375 77.625) (end 164.325 77.625) (width 0.25) (layer "B.Cu") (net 1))
 (segment (start 166.1 78.35) (end 165.375 77.625) (width 0.25) (layer "B.Cu") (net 1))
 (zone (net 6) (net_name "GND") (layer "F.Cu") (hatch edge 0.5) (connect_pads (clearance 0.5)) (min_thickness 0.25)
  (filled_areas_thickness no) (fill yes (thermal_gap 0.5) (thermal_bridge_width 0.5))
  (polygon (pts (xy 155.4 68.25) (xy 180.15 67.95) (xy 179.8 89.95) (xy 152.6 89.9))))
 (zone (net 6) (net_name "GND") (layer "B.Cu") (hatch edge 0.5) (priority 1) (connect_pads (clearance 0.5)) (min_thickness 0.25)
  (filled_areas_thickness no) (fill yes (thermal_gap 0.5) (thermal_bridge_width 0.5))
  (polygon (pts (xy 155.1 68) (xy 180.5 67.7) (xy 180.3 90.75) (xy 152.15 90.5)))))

